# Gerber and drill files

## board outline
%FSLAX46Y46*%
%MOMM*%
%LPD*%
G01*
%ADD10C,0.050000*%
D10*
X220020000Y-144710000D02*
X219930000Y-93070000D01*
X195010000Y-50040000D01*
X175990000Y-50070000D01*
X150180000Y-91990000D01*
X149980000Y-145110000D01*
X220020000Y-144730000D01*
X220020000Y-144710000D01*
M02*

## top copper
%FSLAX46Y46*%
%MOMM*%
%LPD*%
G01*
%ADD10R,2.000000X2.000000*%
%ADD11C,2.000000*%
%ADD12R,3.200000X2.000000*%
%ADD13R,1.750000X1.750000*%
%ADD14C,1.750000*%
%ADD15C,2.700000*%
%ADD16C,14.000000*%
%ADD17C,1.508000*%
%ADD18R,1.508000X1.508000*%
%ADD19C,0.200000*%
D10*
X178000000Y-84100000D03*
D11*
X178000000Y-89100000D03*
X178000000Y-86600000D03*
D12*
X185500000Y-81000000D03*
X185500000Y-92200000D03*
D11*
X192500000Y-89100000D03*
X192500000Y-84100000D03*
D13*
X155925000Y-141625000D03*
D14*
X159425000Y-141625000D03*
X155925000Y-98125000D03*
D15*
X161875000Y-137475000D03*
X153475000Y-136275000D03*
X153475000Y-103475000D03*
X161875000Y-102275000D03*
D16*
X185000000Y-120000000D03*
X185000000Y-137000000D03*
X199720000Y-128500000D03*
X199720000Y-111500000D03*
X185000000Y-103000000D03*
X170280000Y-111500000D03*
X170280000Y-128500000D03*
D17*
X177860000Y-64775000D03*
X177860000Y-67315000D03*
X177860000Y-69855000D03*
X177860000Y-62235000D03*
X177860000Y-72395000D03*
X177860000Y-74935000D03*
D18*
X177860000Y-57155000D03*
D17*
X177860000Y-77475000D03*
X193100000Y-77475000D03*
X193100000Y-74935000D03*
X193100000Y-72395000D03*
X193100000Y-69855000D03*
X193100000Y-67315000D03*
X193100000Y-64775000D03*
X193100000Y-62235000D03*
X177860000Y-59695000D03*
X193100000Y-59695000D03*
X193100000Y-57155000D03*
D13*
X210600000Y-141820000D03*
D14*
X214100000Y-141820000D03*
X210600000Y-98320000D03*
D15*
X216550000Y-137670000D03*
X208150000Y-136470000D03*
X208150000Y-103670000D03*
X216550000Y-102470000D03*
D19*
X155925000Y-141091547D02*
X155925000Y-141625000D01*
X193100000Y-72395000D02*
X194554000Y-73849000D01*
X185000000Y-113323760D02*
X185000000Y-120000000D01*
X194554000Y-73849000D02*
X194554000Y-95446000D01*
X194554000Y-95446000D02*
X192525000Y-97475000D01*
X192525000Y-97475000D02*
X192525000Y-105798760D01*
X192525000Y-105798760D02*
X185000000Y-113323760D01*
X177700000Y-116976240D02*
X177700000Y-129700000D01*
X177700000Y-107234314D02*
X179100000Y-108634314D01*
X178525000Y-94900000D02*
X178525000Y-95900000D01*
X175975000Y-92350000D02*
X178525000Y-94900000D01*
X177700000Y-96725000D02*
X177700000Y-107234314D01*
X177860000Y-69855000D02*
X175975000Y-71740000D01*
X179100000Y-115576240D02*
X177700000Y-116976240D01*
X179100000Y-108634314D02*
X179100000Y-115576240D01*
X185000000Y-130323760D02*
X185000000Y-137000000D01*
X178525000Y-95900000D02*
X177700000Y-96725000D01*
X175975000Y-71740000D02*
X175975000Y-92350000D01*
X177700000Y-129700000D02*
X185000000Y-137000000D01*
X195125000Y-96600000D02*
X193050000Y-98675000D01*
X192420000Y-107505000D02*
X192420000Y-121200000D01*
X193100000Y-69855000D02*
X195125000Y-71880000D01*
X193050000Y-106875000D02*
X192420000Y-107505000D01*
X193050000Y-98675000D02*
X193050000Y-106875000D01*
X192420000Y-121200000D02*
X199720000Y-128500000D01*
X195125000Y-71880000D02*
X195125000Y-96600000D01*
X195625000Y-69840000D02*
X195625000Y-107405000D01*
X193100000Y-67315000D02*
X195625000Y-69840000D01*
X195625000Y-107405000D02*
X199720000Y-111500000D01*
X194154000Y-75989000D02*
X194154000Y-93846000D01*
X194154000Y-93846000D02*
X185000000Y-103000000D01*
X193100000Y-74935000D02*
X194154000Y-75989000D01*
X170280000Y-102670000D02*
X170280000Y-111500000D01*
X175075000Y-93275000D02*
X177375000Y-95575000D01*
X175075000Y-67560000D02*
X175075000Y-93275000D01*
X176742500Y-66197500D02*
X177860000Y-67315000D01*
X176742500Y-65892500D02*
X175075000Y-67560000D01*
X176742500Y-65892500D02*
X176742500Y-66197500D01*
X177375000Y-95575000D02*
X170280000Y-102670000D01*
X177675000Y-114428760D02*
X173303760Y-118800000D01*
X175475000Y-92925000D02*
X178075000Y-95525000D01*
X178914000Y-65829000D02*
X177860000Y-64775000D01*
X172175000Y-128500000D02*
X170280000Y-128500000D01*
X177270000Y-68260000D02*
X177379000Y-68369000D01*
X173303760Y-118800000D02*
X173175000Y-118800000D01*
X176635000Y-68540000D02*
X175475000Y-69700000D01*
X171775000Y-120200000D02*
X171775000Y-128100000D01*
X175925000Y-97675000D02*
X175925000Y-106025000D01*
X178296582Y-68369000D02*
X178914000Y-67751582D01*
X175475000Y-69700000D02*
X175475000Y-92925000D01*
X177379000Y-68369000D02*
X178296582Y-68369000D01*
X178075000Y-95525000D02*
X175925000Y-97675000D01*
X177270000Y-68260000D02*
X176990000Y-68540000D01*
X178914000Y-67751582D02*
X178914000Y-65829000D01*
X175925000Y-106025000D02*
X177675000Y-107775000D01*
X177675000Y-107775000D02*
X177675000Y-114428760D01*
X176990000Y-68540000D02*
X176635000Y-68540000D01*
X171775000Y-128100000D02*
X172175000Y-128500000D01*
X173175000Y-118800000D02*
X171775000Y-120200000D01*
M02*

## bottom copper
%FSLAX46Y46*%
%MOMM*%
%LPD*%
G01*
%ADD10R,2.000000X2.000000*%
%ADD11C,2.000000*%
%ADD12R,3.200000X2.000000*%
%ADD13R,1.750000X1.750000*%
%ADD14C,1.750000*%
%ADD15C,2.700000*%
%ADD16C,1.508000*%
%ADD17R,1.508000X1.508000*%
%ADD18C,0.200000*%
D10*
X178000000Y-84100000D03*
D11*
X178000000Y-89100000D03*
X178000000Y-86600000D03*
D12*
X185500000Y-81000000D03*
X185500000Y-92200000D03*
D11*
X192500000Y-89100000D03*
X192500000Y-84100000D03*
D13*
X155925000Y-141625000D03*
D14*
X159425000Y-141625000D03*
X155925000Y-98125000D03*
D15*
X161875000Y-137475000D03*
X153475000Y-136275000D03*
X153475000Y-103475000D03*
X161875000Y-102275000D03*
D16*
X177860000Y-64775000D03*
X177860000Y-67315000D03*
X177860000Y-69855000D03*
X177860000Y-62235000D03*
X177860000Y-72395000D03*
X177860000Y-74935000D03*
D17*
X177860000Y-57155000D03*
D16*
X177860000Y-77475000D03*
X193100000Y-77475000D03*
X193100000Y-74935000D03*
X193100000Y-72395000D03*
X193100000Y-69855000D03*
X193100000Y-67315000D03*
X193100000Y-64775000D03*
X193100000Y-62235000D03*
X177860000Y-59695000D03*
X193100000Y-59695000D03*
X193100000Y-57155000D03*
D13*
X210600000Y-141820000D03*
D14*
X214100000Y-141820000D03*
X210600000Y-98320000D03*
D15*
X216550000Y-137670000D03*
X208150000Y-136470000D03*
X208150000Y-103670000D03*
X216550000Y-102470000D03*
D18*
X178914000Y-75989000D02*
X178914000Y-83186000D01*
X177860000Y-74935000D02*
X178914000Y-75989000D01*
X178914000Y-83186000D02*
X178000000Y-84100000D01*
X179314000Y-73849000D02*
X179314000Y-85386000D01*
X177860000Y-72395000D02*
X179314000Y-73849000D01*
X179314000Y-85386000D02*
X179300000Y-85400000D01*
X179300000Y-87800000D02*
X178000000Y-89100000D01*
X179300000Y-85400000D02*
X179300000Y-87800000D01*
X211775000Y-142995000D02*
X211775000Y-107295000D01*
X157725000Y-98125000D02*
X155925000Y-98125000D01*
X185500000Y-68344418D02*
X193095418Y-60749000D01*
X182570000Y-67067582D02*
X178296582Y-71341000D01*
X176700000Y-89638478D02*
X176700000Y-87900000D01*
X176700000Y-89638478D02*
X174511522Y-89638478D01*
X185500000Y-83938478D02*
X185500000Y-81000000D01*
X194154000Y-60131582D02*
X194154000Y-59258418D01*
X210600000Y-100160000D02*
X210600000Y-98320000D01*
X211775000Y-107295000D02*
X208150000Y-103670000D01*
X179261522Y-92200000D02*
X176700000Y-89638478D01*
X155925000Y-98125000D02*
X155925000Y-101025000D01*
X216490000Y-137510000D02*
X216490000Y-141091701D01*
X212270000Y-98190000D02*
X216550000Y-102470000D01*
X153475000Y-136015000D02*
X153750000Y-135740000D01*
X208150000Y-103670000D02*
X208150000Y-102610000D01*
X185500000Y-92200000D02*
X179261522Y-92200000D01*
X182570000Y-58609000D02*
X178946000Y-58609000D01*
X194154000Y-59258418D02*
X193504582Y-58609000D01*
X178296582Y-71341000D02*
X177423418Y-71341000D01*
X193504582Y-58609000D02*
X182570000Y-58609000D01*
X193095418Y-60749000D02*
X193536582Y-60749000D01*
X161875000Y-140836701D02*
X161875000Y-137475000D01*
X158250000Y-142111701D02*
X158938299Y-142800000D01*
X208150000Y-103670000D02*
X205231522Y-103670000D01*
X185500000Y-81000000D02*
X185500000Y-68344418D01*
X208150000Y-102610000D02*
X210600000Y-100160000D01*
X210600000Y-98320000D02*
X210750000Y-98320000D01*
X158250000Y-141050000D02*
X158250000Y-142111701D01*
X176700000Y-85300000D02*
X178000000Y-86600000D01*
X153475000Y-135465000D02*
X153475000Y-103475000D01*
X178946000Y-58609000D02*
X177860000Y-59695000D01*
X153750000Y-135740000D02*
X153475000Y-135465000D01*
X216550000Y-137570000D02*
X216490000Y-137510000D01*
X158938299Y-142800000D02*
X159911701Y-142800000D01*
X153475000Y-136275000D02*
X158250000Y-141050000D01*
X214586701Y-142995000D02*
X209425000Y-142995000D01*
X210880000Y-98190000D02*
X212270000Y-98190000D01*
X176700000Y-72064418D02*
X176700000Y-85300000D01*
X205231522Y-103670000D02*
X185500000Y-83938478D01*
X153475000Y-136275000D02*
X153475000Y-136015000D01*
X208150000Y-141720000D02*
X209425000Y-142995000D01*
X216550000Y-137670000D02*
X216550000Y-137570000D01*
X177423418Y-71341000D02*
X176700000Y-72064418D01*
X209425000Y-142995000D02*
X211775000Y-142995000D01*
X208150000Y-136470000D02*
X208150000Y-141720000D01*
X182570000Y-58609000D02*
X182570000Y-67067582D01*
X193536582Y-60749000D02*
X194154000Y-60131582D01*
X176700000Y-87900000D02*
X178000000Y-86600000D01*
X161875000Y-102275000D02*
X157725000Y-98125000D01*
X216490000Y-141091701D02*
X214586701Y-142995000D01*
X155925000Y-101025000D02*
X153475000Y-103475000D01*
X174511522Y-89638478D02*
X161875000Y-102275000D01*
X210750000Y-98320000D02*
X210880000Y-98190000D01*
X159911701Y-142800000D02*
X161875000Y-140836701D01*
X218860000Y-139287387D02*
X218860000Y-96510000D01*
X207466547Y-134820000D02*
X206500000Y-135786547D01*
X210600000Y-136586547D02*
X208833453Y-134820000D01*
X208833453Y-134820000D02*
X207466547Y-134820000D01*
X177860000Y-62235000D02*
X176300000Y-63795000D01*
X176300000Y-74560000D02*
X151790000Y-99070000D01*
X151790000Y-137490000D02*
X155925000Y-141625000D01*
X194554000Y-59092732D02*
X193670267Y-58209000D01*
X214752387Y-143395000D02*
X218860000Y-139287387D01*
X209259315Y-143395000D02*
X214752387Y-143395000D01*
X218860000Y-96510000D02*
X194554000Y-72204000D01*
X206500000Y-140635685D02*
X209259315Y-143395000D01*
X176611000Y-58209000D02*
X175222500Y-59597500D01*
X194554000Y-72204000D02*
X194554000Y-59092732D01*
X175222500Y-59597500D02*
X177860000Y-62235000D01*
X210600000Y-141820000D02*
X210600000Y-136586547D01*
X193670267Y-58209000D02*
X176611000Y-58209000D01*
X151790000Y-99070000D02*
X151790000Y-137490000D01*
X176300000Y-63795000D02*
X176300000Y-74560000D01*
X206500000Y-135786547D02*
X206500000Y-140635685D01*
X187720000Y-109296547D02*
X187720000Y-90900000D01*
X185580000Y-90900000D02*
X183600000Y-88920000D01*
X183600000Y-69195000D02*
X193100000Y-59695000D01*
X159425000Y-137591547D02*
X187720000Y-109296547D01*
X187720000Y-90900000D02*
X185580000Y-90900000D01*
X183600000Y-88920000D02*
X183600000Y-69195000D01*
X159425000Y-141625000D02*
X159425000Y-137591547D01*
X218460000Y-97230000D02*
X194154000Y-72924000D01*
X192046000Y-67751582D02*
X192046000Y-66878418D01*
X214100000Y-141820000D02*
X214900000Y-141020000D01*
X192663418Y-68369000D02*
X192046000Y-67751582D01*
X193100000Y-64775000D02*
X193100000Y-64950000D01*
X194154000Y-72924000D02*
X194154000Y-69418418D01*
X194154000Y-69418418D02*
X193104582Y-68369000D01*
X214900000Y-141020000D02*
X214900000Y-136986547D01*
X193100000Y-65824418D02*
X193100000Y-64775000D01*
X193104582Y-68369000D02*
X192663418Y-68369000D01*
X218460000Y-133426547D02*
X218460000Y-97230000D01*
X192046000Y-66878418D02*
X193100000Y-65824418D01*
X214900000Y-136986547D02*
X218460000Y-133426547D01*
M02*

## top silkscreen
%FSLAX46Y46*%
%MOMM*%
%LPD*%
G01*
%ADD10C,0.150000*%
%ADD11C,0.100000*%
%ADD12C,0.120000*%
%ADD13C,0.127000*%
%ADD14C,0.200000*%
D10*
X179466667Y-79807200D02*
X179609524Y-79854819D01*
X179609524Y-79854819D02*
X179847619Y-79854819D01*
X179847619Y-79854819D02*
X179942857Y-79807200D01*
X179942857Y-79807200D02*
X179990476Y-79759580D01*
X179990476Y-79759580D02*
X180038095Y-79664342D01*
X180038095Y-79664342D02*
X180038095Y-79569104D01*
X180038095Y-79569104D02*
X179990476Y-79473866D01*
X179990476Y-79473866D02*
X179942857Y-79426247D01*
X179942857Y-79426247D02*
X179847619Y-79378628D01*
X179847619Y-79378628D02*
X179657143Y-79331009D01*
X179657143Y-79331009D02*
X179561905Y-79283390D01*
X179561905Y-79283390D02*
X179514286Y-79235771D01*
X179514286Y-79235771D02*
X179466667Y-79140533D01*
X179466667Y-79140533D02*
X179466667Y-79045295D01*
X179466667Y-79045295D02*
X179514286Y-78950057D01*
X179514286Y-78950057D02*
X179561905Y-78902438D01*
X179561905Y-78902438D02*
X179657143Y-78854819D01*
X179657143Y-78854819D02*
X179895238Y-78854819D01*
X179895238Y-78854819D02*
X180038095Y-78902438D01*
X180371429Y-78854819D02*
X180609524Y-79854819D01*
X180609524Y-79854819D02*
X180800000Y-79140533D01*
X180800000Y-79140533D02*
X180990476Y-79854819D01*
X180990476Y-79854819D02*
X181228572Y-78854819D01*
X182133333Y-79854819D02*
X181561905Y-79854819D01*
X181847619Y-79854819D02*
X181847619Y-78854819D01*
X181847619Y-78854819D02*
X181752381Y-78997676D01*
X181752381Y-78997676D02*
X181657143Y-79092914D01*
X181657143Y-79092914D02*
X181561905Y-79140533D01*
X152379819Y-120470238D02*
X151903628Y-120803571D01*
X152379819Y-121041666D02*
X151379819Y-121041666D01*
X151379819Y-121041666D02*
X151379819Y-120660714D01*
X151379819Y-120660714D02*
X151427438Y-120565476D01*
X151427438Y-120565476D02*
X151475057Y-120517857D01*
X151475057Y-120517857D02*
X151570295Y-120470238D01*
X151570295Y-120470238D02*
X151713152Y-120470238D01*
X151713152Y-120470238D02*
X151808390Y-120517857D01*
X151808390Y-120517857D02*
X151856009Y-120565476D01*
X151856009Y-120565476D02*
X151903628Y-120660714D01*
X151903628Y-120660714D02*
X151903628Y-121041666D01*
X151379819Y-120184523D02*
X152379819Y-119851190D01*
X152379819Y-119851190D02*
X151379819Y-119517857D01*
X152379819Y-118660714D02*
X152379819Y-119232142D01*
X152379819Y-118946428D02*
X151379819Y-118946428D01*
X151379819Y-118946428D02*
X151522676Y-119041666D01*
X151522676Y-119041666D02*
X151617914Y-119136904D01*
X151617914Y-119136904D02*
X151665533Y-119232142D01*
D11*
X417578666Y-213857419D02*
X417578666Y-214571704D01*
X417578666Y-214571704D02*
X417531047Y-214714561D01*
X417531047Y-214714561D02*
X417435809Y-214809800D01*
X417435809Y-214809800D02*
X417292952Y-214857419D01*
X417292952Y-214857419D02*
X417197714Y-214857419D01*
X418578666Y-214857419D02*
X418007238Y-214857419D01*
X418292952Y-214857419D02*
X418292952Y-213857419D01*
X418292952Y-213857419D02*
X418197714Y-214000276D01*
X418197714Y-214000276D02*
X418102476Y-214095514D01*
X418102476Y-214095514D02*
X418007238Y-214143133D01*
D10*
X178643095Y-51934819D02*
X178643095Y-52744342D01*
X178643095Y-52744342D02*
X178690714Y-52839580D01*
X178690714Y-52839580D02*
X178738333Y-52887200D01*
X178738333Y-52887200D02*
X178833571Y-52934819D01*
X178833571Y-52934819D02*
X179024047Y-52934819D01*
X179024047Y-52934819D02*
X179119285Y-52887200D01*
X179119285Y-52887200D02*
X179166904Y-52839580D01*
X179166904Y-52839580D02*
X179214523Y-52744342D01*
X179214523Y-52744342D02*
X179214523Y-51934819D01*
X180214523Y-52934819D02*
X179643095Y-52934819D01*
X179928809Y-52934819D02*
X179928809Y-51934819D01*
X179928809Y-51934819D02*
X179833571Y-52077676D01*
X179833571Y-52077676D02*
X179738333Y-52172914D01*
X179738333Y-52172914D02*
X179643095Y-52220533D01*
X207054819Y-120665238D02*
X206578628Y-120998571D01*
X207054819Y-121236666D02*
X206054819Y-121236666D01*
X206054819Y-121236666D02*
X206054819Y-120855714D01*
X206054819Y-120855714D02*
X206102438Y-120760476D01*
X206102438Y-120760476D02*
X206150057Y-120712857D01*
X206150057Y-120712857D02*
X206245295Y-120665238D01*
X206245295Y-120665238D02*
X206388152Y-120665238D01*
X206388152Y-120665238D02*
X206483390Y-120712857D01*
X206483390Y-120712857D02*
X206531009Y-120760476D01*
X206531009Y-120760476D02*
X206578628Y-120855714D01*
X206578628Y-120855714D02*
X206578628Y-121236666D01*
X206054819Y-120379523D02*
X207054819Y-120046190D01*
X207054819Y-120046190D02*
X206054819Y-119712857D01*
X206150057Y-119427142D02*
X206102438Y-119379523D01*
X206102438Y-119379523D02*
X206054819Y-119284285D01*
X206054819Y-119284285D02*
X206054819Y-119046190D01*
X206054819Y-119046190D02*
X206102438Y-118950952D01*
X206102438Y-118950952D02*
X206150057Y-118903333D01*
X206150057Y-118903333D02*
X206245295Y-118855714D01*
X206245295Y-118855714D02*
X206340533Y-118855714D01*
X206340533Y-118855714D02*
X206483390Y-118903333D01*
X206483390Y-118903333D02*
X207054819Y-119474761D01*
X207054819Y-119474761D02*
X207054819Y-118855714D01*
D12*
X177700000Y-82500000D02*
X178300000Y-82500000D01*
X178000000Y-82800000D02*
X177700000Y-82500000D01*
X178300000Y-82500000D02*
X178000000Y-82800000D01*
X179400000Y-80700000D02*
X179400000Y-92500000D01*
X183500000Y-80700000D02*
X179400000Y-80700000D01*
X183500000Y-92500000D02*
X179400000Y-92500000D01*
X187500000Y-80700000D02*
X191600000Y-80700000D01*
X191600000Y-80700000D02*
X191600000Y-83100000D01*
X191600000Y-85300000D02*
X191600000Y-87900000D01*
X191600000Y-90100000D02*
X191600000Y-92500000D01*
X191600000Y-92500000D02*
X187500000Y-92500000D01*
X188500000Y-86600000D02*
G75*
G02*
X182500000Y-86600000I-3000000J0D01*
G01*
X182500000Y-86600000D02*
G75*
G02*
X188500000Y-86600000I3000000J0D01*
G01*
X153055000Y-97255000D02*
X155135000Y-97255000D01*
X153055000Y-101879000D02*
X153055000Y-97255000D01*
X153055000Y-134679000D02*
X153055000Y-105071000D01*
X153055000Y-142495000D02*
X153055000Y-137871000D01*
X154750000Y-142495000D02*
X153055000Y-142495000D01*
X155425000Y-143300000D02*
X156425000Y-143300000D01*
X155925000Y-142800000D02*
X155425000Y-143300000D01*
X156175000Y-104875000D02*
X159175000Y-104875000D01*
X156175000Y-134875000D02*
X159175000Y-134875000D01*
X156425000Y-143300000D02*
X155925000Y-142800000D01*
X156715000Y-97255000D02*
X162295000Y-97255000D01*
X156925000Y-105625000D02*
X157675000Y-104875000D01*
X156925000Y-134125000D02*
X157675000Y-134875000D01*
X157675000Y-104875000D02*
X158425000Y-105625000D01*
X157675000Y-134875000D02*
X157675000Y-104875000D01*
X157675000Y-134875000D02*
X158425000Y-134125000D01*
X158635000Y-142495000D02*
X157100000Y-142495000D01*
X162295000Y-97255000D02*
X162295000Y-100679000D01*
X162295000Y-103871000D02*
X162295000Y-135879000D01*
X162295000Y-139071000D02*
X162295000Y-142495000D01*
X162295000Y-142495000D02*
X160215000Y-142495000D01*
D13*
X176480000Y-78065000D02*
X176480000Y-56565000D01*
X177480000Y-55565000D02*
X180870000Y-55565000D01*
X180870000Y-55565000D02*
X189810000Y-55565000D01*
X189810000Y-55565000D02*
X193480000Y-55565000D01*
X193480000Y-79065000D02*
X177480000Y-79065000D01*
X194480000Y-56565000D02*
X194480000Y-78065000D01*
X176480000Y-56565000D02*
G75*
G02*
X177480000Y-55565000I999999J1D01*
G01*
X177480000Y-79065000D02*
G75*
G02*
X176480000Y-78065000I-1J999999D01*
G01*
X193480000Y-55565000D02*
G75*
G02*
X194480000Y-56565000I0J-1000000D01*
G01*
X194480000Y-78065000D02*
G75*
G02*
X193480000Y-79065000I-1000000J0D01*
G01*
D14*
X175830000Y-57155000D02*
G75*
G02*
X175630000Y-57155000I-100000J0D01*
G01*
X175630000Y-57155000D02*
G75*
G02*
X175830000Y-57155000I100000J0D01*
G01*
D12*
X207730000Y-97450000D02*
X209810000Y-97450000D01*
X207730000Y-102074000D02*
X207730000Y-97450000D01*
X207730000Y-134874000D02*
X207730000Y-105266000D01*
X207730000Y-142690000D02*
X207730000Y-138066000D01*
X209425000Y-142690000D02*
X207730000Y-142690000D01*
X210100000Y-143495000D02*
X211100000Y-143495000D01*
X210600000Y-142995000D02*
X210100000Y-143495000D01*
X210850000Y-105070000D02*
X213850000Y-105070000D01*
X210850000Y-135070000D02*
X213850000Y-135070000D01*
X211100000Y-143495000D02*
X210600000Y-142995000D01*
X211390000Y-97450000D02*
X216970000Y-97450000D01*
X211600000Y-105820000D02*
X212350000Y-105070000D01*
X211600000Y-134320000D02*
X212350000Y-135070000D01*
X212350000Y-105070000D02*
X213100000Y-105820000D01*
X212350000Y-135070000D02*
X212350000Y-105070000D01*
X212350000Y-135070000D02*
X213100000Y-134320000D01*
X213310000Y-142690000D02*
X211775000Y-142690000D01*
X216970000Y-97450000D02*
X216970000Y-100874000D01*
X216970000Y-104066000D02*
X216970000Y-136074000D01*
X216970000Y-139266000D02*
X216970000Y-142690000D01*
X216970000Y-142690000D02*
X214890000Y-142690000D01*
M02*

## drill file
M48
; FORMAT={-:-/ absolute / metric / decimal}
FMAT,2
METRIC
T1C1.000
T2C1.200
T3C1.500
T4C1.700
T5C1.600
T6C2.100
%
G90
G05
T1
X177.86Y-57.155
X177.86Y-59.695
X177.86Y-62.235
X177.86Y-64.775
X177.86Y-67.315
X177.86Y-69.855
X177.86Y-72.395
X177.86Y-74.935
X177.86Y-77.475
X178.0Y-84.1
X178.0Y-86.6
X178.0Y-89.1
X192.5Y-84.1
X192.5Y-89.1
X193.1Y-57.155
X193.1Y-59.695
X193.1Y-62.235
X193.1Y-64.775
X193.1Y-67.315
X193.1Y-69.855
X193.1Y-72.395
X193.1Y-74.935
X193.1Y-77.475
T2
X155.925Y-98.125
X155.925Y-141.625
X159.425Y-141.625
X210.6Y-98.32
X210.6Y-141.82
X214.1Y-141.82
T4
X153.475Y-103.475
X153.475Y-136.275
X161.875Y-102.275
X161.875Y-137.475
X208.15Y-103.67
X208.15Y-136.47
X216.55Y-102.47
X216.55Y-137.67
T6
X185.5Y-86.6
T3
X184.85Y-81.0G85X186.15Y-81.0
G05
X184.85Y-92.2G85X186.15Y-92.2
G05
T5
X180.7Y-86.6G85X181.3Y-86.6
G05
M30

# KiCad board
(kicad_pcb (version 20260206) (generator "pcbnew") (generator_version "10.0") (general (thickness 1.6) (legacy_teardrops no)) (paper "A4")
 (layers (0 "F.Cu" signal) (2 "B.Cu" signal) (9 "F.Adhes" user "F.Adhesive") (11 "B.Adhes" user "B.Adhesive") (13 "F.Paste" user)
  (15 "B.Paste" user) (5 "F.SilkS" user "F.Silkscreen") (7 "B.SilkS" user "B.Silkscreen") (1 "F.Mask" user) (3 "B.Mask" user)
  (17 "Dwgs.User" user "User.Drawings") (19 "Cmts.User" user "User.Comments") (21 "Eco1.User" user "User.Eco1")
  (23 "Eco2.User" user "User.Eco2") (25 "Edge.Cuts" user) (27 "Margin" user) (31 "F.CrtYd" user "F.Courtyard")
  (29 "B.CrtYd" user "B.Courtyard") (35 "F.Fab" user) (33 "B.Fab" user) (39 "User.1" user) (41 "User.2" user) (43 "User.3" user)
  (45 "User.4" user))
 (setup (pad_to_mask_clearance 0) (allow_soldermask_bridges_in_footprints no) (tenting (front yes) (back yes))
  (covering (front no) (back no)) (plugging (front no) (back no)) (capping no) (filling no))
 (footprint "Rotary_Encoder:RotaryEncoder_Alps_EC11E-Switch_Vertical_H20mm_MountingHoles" (layer "F.Cu") (at 178 84.1)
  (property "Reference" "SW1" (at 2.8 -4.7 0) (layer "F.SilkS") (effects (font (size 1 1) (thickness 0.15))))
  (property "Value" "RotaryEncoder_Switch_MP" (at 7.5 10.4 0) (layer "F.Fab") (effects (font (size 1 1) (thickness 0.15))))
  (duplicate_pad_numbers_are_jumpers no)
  (fp_line (start -0.3 -1.6) (end 0.3 -1.6) (stroke (width 0.12) (type solid)) (layer "F.SilkS"))
  (fp_line (start 0 -1.3) (end -0.3 -1.6) (stroke (width 0.12) (type solid)) (layer "F.SilkS"))
  (fp_line (start 0.3 -1.6) (end 0 -1.3) (stroke (width 0.12) (type solid)) (layer "F.SilkS"))
  (fp_line (start 1.4 -3.4) (end 1.4 8.4) (stroke (width 0.12) (type solid)) (layer "F.SilkS"))
  (fp_line (start 5.5 -3.4) (end 1.4 -3.4) (stroke (width 0.12) (type solid)) (layer "F.SilkS"))
  (fp_line (start 5.5 8.4) (end 1.4 8.4) (stroke (width 0.12) (type solid)) (layer "F.SilkS"))
  (fp_line (start 9.5 -3.4) (end 13.6 -3.4) (stroke (width 0.12) (type solid)) (layer "F.SilkS"))
  (fp_line (start 13.6 -3.4) (end 13.6 -1) (stroke (width 0.12) (type solid)) (layer "F.SilkS"))
  (fp_line (start 13.6 1.2) (end 13.6 3.8) (stroke (width 0.12) (type solid)) (layer "F.SilkS"))
  (fp_line (start 13.6 6) (end 13.6 8.4) (stroke (width 0.12) (type solid)) (layer "F.SilkS"))
  (fp_line (start 13.6 8.4) (end 9.5 8.4) (stroke (width 0.12) (type solid)) (layer "F.SilkS"))
  (fp_circle (center 7.5 2.5) (end 10.5 2.5) (stroke (width 0.12) (type solid)) (fill no) (layer "F.SilkS"))
  (pad "" np_thru_hole oval (at 3 2.5) (size 2.2 1.6) (drill oval 2.2 1.6) (layers "*.Mask"))
  (pad "" np_thru_hole circle (at 7.5 2.5) (size 2.1 2.1) (drill 2.1) (layers "*.Mask"))
  (pad "A" thru_hole rect (at 0 0) (size 2 2) (drill 1) (layers "*.Cu" "*.Mask") (remove_unused_layers no) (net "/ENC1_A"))
  (pad "B" thru_hole circle (at 0 5) (size 2 2) (drill 1) (layers "*.Cu" "*.Mask") (remove_unused_layers no) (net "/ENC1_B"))
  (pad "C" thru_hole circle (at 0 2.5) (size 2 2) (drill 1) (layers "*.Cu" "*.Mask") (remove_unused_layers no) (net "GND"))
  (pad "MP" thru_hole rect (at 7.5 -3.1) (size 3.2 2) (drill oval 2.8 1.5) (layers "*.Cu" "*.Mask") (remove_unused_layers no) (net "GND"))
  (pad "MP" thru_hole rect (at 7.5 8.1) (size 3.2 2) (drill oval 2.8 1.5) (layers "*.Cu" "*.Mask") (remove_unused_layers no) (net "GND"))
  (pad "S1" thru_hole circle (at 14.5 5) (size 2 2) (drill 1) (layers "*.Cu" "*.Mask") (remove_unused_layers no)
   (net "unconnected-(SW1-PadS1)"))
  (pad "S2" thru_hole circle (at 14.5 0) (size 2 2) (drill 1) (layers "*.Cu" "*.Mask") (remove_unused_layers no)
   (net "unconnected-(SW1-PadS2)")))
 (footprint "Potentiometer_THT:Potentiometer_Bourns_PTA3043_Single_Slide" (layer "F.Cu") (at 155.925 141.625 90)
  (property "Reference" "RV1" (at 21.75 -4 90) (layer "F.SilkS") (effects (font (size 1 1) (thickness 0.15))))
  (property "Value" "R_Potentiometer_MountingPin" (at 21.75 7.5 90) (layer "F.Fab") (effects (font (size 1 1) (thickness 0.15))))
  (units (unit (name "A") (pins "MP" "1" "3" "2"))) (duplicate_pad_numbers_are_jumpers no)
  (fp_line (start 44.37 -2.87) (end 44.37 -0.79) (stroke (width 0.12) (type solid)) (layer "F.SilkS"))
  (fp_line (start 39.746 -2.87) (end 44.37 -2.87) (stroke (width 0.12) (type solid)) (layer "F.SilkS"))
  (fp_line (start 6.946 -2.87) (end 36.554 -2.87) (stroke (width 0.12) (type solid)) (layer "F.SilkS"))
  (fp_line (start -0.87 -2.87) (end 3.754 -2.87) (stroke (width 0.12) (type solid)) (layer "F.SilkS"))
  (fp_line (start -0.87 -1.175) (end -0.87 -2.87) (stroke (width 0.12) (type solid)) (layer "F.SilkS"))
  (fp_line (start -1.675 -0.5) (end -1.675 0.5) (stroke (width 0.12) (type solid)) (layer "F.SilkS"))
  (fp_line (start -1.175 0) (end -1.675 -0.5) (stroke (width 0.12) (type solid)) (layer "F.SilkS"))
  (fp_line (start 36.75 0.25) (end 36.75 3.25) (stroke (width 0.12) (type solid)) (layer "F.SilkS"))
  (fp_line (start 6.75 0.25) (end 6.75 3.25) (stroke (width 0.12) (type solid)) (layer "F.SilkS"))
  (fp_line (start -1.675 0.5) (end -1.175 0) (stroke (width 0.12) (type solid)) (layer "F.SilkS"))
  (fp_line (start 44.37 0.79) (end 44.37 6.37) (stroke (width 0.12) (type solid)) (layer "F.SilkS"))
  (fp_line (start 36 1) (end 36.75 1.75) (stroke (width 0.12) (type solid)) (layer "F.SilkS"))
  (fp_line (start 7.5 1) (end 6.75 1.75) (stroke (width 0.12) (type solid)) (layer "F.SilkS"))
  (fp_line (start 36.75 1.75) (end 36 2.5) (stroke (width 0.12) (type solid)) (layer "F.SilkS"))
  (fp_line (start 6.75 1.75) (end 36.75 1.75) (stroke (width 0.12) (type solid)) (layer "F.SilkS"))
  (fp_line (start 6.75 1.75) (end 7.5 2.5) (stroke (width 0.12) (type solid)) (layer "F.SilkS"))
  (fp_line (start -0.87 2.71) (end -0.87 1.175) (stroke (width 0.12) (type solid)) (layer "F.SilkS"))
  (fp_line (start 44.37 6.37) (end 40.946 6.37) (stroke (width 0.12) (type solid)) (layer "F.SilkS"))
  (fp_line (start 37.754 6.37) (end 5.746 6.37) (stroke (width 0.12) (type solid)) (layer "F.SilkS"))
  (fp_line (start 2.554 6.37) (end -0.87 6.37) (stroke (width 0.12) (type solid)) (layer "F.SilkS"))
  (fp_line (start -0.87 6.37) (end -0.87 4.29) (stroke (width 0.12) (type solid)) (layer "F.SilkS"))
  (pad "1" thru_hole rect (at 0 0 90) (size 1.75 1.75) (drill 1.2) (layers "*.Cu" "*.Mask") (remove_unused_layers no) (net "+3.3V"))
  (pad "2" thru_hole circle (at 0 3.5 90) (size 1.75 1.75) (drill 1.2) (layers "*.Cu" "*.Mask") (remove_unused_layers no) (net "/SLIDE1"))
  (pad "3" thru_hole circle (at 43.5 0 90) (size 1.75 1.75) (drill 1.2) (layers "*.Cu" "*.Mask") (remove_unused_layers no) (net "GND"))
  (pad "MP" thru_hole circle (at 4.15 5.95 90) (size 2.7 2.7) (drill 1.7) (layers "*.Cu" "*.Mask") (remove_unused_layers no) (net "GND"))
  (pad "MP" thru_hole circle (at 5.35 -2.45 90) (size 2.7 2.7) (drill 1.7) (layers "*.Cu" "*.Mask") (remove_unused_layers no) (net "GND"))
  (pad "MP" thru_hole circle (at 38.15 -2.45 90) (size 2.7 2.7) (drill 1.7) (layers "*.Cu" "*.Mask") (remove_unused_layers no) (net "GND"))
  (pad "MP" thru_hole circle (at 39.35 5.95 90) (size 2.7 2.7) (drill 1.7) (layers "*.Cu" "*.Mask") (remove_unused_layers no) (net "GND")))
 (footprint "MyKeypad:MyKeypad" (layer "F.Cu") (at 407 226)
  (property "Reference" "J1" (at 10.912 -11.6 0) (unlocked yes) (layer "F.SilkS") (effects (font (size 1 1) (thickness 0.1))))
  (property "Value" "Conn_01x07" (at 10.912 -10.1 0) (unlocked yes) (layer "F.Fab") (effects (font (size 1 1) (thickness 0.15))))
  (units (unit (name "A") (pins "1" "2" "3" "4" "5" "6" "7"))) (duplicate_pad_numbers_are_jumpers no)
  (pad "1" smd circle (at -222 -106 120) (size 14 14) (layers "F.Cu" "F.Mask") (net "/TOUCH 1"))
  (pad "2" smd circle (at -222 -89 120) (size 14 14) (layers "F.Cu" "F.Mask") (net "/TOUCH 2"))
  (pad "3" smd circle (at -207.28 -97.5 120) (size 14 14) (layers "F.Cu" "F.Mask") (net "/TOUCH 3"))
  (pad "4" smd circle (at -207.28 -114.5 120) (size 14 14) (layers "F.Cu" "F.Mask") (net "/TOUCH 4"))
  (pad "5" smd circle (at -222 -123 120) (size 14 14) (layers "F.Cu" "F.Mask") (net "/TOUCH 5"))
  (pad "6" smd circle (at -236.72 -114.5 120) (size 14 14) (layers "F.Cu" "F.Mask") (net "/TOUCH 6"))
  (pad "7" smd circle (at -236.72 -97.5 120) (size 14 14) (layers "F.Cu" "F.Mask") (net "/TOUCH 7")))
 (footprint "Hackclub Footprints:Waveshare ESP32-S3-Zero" (layer "F.Cu") (at 185.48 67.315)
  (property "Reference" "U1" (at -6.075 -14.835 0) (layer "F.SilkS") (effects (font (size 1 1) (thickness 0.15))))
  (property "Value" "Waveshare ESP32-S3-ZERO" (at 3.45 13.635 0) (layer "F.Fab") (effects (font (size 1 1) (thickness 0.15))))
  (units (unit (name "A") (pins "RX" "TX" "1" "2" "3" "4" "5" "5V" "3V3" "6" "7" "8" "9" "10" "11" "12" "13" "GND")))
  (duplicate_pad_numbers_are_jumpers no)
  (fp_line (start -9 10.75) (end -9 -10.75) (stroke (width 0.127) (type solid)) (layer "F.SilkS"))
  (fp_line (start -8 -11.75) (end -4.61 -11.75) (stroke (width 0.127) (type solid)) (layer "F.SilkS"))
  (fp_line (start -4.61 -11.75) (end 4.33 -11.75) (stroke (width 0.127) (type solid)) (layer "F.SilkS"))
  (fp_line (start 4.33 -11.75) (end 8 -11.75) (stroke (width 0.127) (type solid)) (layer "F.SilkS"))
  (fp_line (start 8 11.75) (end -8 11.75) (stroke (width 0.127) (type solid)) (layer "F.SilkS"))
  (fp_line (start 9 -10.75) (end 9 10.75) (stroke (width 0.127) (type solid)) (layer "F.SilkS"))
  (fp_arc (start -9 -10.75) (mid -8.707107 -11.457107) (end -8 -11.75) (stroke (width 0.127) (type solid)) (layer "F.SilkS"))
  (fp_arc (start -8 11.75) (mid -8.707107 11.457107) (end -9 10.75) (stroke (width 0.127) (type solid)) (layer "F.SilkS"))
  (fp_arc (start 8 -11.75) (mid 8.707107 -11.457107) (end 9 -10.75) (stroke (width 0.127) (type solid)) (layer "F.SilkS"))
  (fp_arc (start 9 10.75) (mid 8.707107 11.457107) (end 8 11.75) (stroke (width 0.127) (type solid)) (layer "F.SilkS"))
  (fp_circle (center -9.75 -10.16) (end -9.65 -10.16) (stroke (width 0.2) (type solid)) (fill no) (layer "F.SilkS"))
  (pad "1" thru_hole circle (at -7.62 -2.54) (size 1.508 1.508) (drill 1) (layers "*.Cu" "*.Mask") (remove_unused_layers no)
   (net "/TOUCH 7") (solder_mask_margin 0.102))
  (pad "2" thru_hole circle (at -7.62 0) (size 1.508 1.508) (drill 1) (layers "*.Cu" "*.Mask") (remove_unused_layers no) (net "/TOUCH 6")
   (solder_mask_margin 0.102))
  (pad "3" thru_hole circle (at -7.62 2.54) (size 1.508 1.508) (drill 1) (layers "*.Cu" "*.Mask") (remove_unused_layers no) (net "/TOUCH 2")
   (solder_mask_margin 0.102))
  (pad "3V3" thru_hole circle (at -7.62 -5.08) (size 1.508 1.508) (drill 1) (layers "*.Cu" "*.Mask") (remove_unused_layers no) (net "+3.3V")
   (solder_mask_margin 0.102))
  (pad "4" thru_hole circle (at -7.62 5.08) (size 1.508 1.508) (drill 1) (layers "*.Cu" "*.Mask") (remove_unused_layers no) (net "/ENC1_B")
   (solder_mask_margin 0.102))
  (pad "5" thru_hole circle (at -7.62 7.62) (size 1.508 1.508) (drill 1) (layers "*.Cu" "*.Mask") (remove_unused_layers no) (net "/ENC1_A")
   (solder_mask_margin 0.102))
  (pad "5V" thru_hole rect (at -7.62 -10.16) (size 1.508 1.508) (drill 1) (layers "*.Cu" "*.Mask") (remove_unused_layers no) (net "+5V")
   (solder_mask_margin 0.102))
  (pad "6" thru_hole circle (at -7.62 10.16) (size 1.508 1.508) (drill 1) (layers "*.Cu" "*.Mask") (remove_unused_layers no)
   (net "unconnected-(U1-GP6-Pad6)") (solder_mask_margin 0.102))
  (pad "7" thru_hole circle (at 7.62 10.16) (size 1.508 1.508) (drill 1) (layers "*.Cu" "*.Mask") (remove_unused_layers no)
   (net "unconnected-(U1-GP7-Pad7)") (solder_mask_margin 0.102))
  (pad "8" thru_hole circle (at 7.62 7.62) (size 1.508 1.508) (drill 1) (layers "*.Cu" "*.Mask") (remove_unused_layers no) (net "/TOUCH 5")
   (solder_mask_margin 0.102))
  (pad "9" thru_hole circle (at 7.62 5.08) (size 1.508 1.508) (drill 1) (layers "*.Cu" "*.Mask") (remove_unused_layers no) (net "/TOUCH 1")
   (solder_mask_margin 0.102))
  (pad "10" thru_hole circle (at 7.62 2.54) (size 1.508 1.508) (drill 1) (layers "*.Cu" "*.Mask") (remove_unused_layers no) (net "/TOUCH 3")
   (solder_mask_margin 0.102))
  (pad "11" thru_hole circle (at 7.62 0) (size 1.508 1.508) (drill 1) (layers "*.Cu" "*.Mask") (remove_unused_layers no) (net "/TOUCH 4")
   (solder_mask_margin 0.102))
  (pad "12" thru_hole circle (at 7.62 -2.54) (size 1.508 1.508) (drill 1) (layers "*.Cu" "*.Mask") (remove_unused_layers no) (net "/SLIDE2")
   (solder_mask_margin 0.102))
  (pad "13" thru_hole circle (at 7.62 -5.08) (size 1.508 1.508) (drill 1) (layers "*.Cu" "*.Mask") (remove_unused_layers no)
   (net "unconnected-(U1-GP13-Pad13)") (solder_mask_margin 0.102))
  (pad "GND" thru_hole circle (at -7.62 -7.62) (size 1.508 1.508) (drill 1) (layers "*.Cu" "*.Mask") (remove_unused_layers no) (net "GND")
   (solder_mask_margin 0.102))
  (pad "RX" thru_hole circle (at 7.62 -7.62) (size 1.508 1.508) (drill 1) (layers "*.Cu" "*.Mask") (remove_unused_layers no) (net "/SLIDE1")
   (solder_mask_margin 0.102))
  (pad "TX" thru_hole circle (at 7.62 -10.16) (size 1.508 1.508) (drill 1) (layers "*.Cu" "*.Mask") (remove_unused_layers no)
   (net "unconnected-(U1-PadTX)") (solder_mask_margin 0.102)))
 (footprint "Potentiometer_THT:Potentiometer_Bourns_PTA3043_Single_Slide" (layer "F.Cu") (at 210.6 141.82 90)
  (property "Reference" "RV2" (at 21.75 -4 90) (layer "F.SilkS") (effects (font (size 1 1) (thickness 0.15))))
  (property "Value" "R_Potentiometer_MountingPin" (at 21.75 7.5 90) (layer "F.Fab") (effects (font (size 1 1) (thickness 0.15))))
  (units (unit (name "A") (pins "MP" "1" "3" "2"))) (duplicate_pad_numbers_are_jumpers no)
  (fp_line (start 44.37 -2.87) (end 44.37 -0.79) (stroke (width 0.12) (type solid)) (layer "F.SilkS"))
  (fp_line (start 39.746 -2.87) (end 44.37 -2.87) (stroke (width 0.12) (type solid)) (layer "F.SilkS"))
  (fp_line (start 6.946 -2.87) (end 36.554 -2.87) (stroke (width 0.12) (type solid)) (layer "F.SilkS"))
  (fp_line (start -0.87 -2.87) (end 3.754 -2.87) (stroke (width 0.12) (type solid)) (layer "F.SilkS"))
  (fp_line (start -0.87 -1.175) (end -0.87 -2.87) (stroke (width 0.12) (type solid)) (layer "F.SilkS"))
  (fp_line (start -1.675 -0.5) (end -1.675 0.5) (stroke (width 0.12) (type solid)) (layer "F.SilkS"))
  (fp_line (start -1.175 0) (end -1.675 -0.5) (stroke (width 0.12) (type solid)) (layer "F.SilkS"))
  (fp_line (start 36.75 0.25) (end 36.75 3.25) (stroke (width 0.12) (type solid)) (layer "F.SilkS"))
  (fp_line (start 6.75 0.25) (end 6.75 3.25) (stroke (width 0.12) (type solid)) (layer "F.SilkS"))
  (fp_line (start -1.675 0.5) (end -1.175 0) (stroke (width 0.12) (type solid)) (layer "F.SilkS"))
  (fp_line (start 44.37 0.79) (end 44.37 6.37) (stroke (width 0.12) (type solid)) (layer "F.SilkS"))
  (fp_line (start 36 1) (end 36.75 1.75) (stroke (width 0.12) (type solid)) (layer "F.SilkS"))
  (fp_line (start 7.5 1) (end 6.75 1.75) (stroke (width 0.12) (type solid)) (layer "F.SilkS"))
  (fp_line (start 36.75 1.75) (end 36 2.5) (stroke (width 0.12) (type solid)) (layer "F.SilkS"))
  (fp_line (start 6.75 1.75) (end 36.75 1.75) (stroke (width 0.12) (type solid)) (layer "F.SilkS"))
  (fp_line (start 6.75 1.75) (end 7.5 2.5) (stroke (width 0.12) (type solid)) (layer "F.SilkS"))
  (fp_line (start -0.87 2.71) (end -0.87 1.175) (stroke (width 0.12) (type solid)) (layer "F.SilkS"))
  (fp_line (start 44.37 6.37) (end 40.946 6.37) (stroke (width 0.12) (type solid)) (layer "F.SilkS"))
  (fp_line (start 37.754 6.37) (end 5.746 6.37) (stroke (width 0.12) (type solid)) (layer "F.SilkS"))
  (fp_line (start 2.554 6.37) (end -0.87 6.37) (stroke (width 0.12) (type solid)) (layer "F.SilkS"))
  (fp_line (start -0.87 6.37) (end -0.87 4.29) (stroke (width 0.12) (type solid)) (layer "F.SilkS"))
  (pad "1" thru_hole rect (at 0 0 90) (size 1.75 1.75) (drill 1.2) (layers "*.Cu" "*.Mask") (remove_unused_layers no) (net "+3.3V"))
  (pad "2" thru_hole circle (at 0 3.5 90) (size 1.75 1.75) (drill 1.2) (layers "*.Cu" "*.Mask") (remove_unused_layers no) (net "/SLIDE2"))
  (pad "3" thru_hole circle (at 43.5 0 90) (size 1.75 1.75) (drill 1.2) (layers "*.Cu" "*.Mask") (remove_unused_layers no) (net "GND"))
  (pad "MP" thru_hole circle (at 4.15 5.95 90) (size 2.7 2.7) (drill 1.7) (layers "*.Cu" "*.Mask") (remove_unused_layers no) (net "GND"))
  (pad "MP" thru_hole circle (at 5.35 -2.45 90) (size 2.7 2.7) (drill 1.7) (layers "*.Cu" "*.Mask") (remove_unused_layers no) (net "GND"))
  (pad "MP" thru_hole circle (at 38.15 -2.45 90) (size 2.7 2.7) (drill 1.7) (layers "*.Cu" "*.Mask") (remove_unused_layers no) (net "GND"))
  (pad "MP" thru_hole circle (at 39.35 5.95 90) (size 2.7 2.7) (drill 1.7) (layers "*.Cu" "*.Mask") (remove_unused_layers no) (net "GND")))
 (gr_poly
  (pts (xy 220.02 144.71) (xy 219.93 93.07) (xy 195.01 50.04) (xy 175.99 50.07) (xy 150.18 91.99) (xy 149.98 145.11) (xy 220.02 144.73))
  (stroke (width 0.05) (type solid)) (fill no) (layer "Edge.Cuts"))
 (segment (start 178.914 75.989) (end 178.914 83.186) (width 0.2) (layer "B.Cu") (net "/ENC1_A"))
 (segment (start 177.86 74.935) (end 178.914 75.989) (width 0.2) (layer "B.Cu") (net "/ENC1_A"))
 (segment (start 178.914 83.186) (end 178 84.1) (width 0.2) (layer "B.Cu") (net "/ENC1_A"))
 (segment (start 179.314 73.849) (end 179.314 85.386) (width 0.2) (layer "B.Cu") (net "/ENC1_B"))
 (segment (start 177.86 72.395) (end 179.314 73.849) (width 0.2) (layer "B.Cu") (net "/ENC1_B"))
 (segment (start 179.314 85.386) (end 179.3 85.4) (width 0.2) (layer "B.Cu") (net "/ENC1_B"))
 (segment (start 179.3 87.8) (end 178 89.1) (width 0.2) (layer "B.Cu") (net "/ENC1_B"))
 (segment (start 179.3 85.4) (end 179.3 87.8) (width 0.2) (layer "B.Cu") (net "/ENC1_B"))
 (segment (start 211.775 142.995) (end 211.775 107.295) (width 0.2) (layer "B.Cu") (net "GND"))
 (segment (start 157.725 98.125) (end 155.925 98.125) (width 0.2) (layer "B.Cu") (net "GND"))
 (segment (start 185.5 68.344418) (end 193.095418 60.749) (width 0.2) (layer "B.Cu") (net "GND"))
 (segment (start 182.57 67.067582) (end 178.296582 71.341) (width 0.2) (layer "B.Cu") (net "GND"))
 (segment (start 176.7 89.638478) (end 176.7 87.9) (width 0.2) (layer "B.Cu") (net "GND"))
 (segment (start 176.7 89.638478) (end 174.511522 89.638478) (width 0.2) (layer "B.Cu") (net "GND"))
 (segment (start 185.5 83.938478) (end 185.5 81) (width 0.2) (layer "B.Cu") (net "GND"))
 (segment (start 194.154 60.131582) (end 194.154 59.258418) (width 0.2) (layer "B.Cu") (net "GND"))
 (segment (start 210.6 100.16) (end 210.6 98.32) (width 0.2) (layer "B.Cu") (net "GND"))
 (segment (start 211.775 107.295) (end 208.15 103.67) (width 0.2) (layer "B.Cu") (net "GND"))
 (segment (start 179.261522 92.2) (end 176.7 89.638478) (width 0.2) (layer "B.Cu") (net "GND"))
 (segment (start 155.925 98.125) (end 155.925 101.025) (width 0.2) (layer "B.Cu") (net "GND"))
 (segment (start 216.49 137.51) (end 216.49 141.091701) (width 0.2) (layer "B.Cu") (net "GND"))
 (segment (start 212.27 98.19) (end 216.55 102.47) (width 0.2) (layer "B.Cu") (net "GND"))
 (segment (start 153.475 136.015) (end 153.75 135.74) (width 0.2) (layer "B.Cu") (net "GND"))
 (segment (start 208.15 103.67) (end 208.15 102.61) (width 0.2) (layer "B.Cu") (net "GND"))
 (segment (start 185.5 92.2) (end 179.261522 92.2) (width 0.2) (layer "B.Cu") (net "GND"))
 (segment (start 182.57 58.609) (end 178.946 58.609) (width 0.2) (layer "B.Cu") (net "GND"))
 (segment (start 194.154 59.258418) (end 193.504582 58.609) (width 0.2) (layer "B.Cu") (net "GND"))
 (segment (start 178.296582 71.341) (end 177.423418 71.341) (width 0.2) (layer "B.Cu") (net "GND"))
 (segment (start 193.504582 58.609) (end 182.57 58.609) (width 0.2) (layer "B.Cu") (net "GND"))
 (segment (start 193.095418 60.749) (end 193.536582 60.749) (width 0.2) (layer "B.Cu") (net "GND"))
 (segment (start 161.875 140.836701) (end 161.875 137.475) (width 0.2) (layer "B.Cu") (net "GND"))
 (segment (start 158.25 142.111701) (end 158.938299 142.8) (width 0.2) (layer "B.Cu") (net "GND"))
 (segment (start 208.15 103.67) (end 205.231522 103.67) (width 0.2) (layer "B.Cu") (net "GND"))
 (segment (start 185.5 81) (end 185.5 68.344418) (width 0.2) (layer "B.Cu") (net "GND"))
 (segment (start 208.15 102.61) (end 210.6 100.16) (width 0.2) (layer "B.Cu") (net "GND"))
 (segment (start 210.6 98.32) (end 210.75 98.32) (width 0.2) (layer "B.Cu") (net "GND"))
 (segment (start 158.25 141.05) (end 158.25 142.111701) (width 0.2) (layer "B.Cu") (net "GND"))
 (segment (start 176.7 85.3) (end 178 86.6) (width 0.2) (layer "B.Cu") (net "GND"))
 (segment (start 153.475 135.465) (end 153.475 103.475) (width 0.2) (layer "B.Cu") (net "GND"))
 (segment (start 178.946 58.609) (end 177.86 59.695) (width 0.2) (layer "B.Cu") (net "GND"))
 (segment (start 153.75 135.74) (end 153.475 135.465) (width 0.2) (layer "B.Cu") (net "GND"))
 (segment (start 216.55 137.57) (end 216.49 137.51) (width 0.2) (layer "B.Cu") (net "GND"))
 (segment (start 158.938299 142.8) (end 159.911701 142.8) (width 0.2) (layer "B.Cu") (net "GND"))
 (segment (start 153.475 136.275) (end 158.25 141.05) (width 0.2) (layer "B.Cu") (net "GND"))
 (segment (start 214.586701 142.995) (end 209.425 142.995) (width 0.2) (layer "B.Cu") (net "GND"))
 (segment (start 210.88 98.19) (end 212.27 98.19) (width 0.2) (layer "B.Cu") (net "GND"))
 (segment (start 176.7 72.064418) (end 176.7 85.3) (width 0.2) (layer "B.Cu") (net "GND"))
 (segment (start 205.231522 103.67) (end 185.5 83.938478) (width 0.2) (layer "B.Cu") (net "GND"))
 (segment (start 153.475 136.275) (end 153.475 136.015) (width 0.2) (layer "B.Cu") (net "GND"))
 (segment (start 208.15 141.72) (end 209.425 142.995) (width 0.2) (layer "B.Cu") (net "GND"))
 (segment (start 216.55 137.67) (end 216.55 137.57) (width 0.2) (layer "B.Cu") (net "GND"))
 (segment (start 177.423418 71.341) (end 176.7 72.064418) (width 0.2) (layer "B.Cu") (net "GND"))
 (segment (start 209.425 142.995) (end 211.775 142.995) (width 0.2) (layer "B.Cu") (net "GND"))
 (segment (start 208.15 136.47) (end 208.15 141.72) (width 0.2) (layer "B.Cu") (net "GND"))
 (segment (start 182.57 58.609) (end 182.57 67.067582) (width 0.2) (layer "B.Cu") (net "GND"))
 (segment (start 193.536582 60.749) (end 194.154 60.131582) (width 0.2) (layer "B.Cu") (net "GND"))
 (segment (start 176.7 87.9) (end 178 86.6) (width 0.2) (layer "B.Cu") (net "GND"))
 (segment (start 161.875 102.275) (end 157.725 98.125) (width 0.2) (layer "B.Cu") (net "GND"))
 (segment (start 216.49 141.091701) (end 214.586701 142.995) (width 0.2) (layer "B.Cu") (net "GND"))
 (segment (start 155.925 101.025) (end 153.475 103.475) (width 0.2) (layer "B.Cu") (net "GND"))
 (segment (start 174.511522 89.638478) (end 161.875 102.275) (width 0.2) (layer "B.Cu") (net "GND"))
 (segment (start 210.75 98.32) (end 210.88 98.19) (width 0.2) (layer "B.Cu") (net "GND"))
 (segment (start 159.911701 142.8) (end 161.875 140.836701) (width 0.2) (layer "B.Cu") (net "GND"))
 (segment (start 155.925 141.091547) (end 155.925 141.625) (width 0.2) (layer "F.Cu") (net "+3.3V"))
 (segment (start 218.86 139.287387) (end 218.86 96.51) (width 0.2) (layer "B.Cu") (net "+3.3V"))
 (segment (start 207.466547 134.82) (end 206.5 135.786547) (width 0.2) (layer "B.Cu") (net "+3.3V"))
 (segment (start 210.6 136.586547) (end 208.833453 134.82) (width 0.2) (layer "B.Cu") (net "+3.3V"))
 (segment (start 208.833453 134.82) (end 207.466547 134.82) (width 0.2) (layer "B.Cu") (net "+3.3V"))
 (segment (start 177.86 62.235) (end 176.3 63.795) (width 0.2) (layer "B.Cu") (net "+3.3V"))
 (segment (start 176.3 74.56) (end 151.79 99.07) (width 0.2) (layer "B.Cu") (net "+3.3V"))
 (segment (start 151.79 137.49) (end 155.925 141.625) (width 0.2) (layer "B.Cu") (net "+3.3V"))
 (segment (start 194.554 59.092732) (end 193.670267 58.209) (width 0.2) (layer "B.Cu") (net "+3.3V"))
 (segment (start 214.752387 143.395) (end 218.86 139.287387) (width 0.2) (layer "B.Cu") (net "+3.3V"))
 (segment (start 209.259315 143.395) (end 214.752387 143.395) (width 0.2) (layer "B.Cu") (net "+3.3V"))
 (segment (start 218.86 96.51) (end 194.554 72.204) (width 0.2) (layer "B.Cu") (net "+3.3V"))
 (segment (start 206.5 140.635685) (end 209.259315 143.395) (width 0.2) (layer "B.Cu") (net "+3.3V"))
 (segment (start 176.611 58.209) (end 175.2225 59.5975) (width 0.2) (layer "B.Cu") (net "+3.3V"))
 (segment (start 194.554 72.204) (end 194.554 59.092732) (width 0.2) (layer "B.Cu") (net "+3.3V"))
 (segment (start 175.2225 59.5975) (end 177.86 62.235) (width 0.2) (layer "B.Cu") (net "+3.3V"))
 (segment (start 210.6 141.82) (end 210.6 136.586547) (width 0.2) (layer "B.Cu") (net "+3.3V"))
 (segment (start 193.670267 58.209) (end 176.611 58.209) (width 0.2) (layer "B.Cu") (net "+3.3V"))
 (segment (start 151.79 99.07) (end 151.79 137.49) (width 0.2) (layer "B.Cu") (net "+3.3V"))
 (segment (start 176.3 63.795) (end 176.3 74.56) (width 0.2) (layer "B.Cu") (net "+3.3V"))
 (segment (start 206.5 135.786547) (end 206.5 140.635685) (width 0.2) (layer "B.Cu") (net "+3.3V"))
 (segment (start 187.72 109.296547) (end 187.72 90.9) (width 0.2) (layer "B.Cu") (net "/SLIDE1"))
 (segment (start 185.58 90.9) (end 183.6 88.92) (width 0.2) (layer "B.Cu") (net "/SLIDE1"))
 (segment (start 183.6 69.195) (end 193.1 59.695) (width 0.2) (layer "B.Cu") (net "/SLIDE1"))
 (segment (start 159.425 137.591547) (end 187.72 109.296547) (width 0.2) (layer "B.Cu") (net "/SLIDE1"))
 (segment (start 187.72 90.9) (end 185.58 90.9) (width 0.2) (layer "B.Cu") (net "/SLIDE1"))
 (segment (start 183.6 88.92) (end 183.6 69.195) (width 0.2) (layer "B.Cu") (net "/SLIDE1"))
 (segment (start 159.425 141.625) (end 159.425 137.591547) (width 0.2) (layer "B.Cu") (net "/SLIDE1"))
 (segment (start 193.1 72.395) (end 194.554 73.849) (width 0.2) (layer "F.Cu") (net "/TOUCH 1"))
 (segment (start 185 113.32376) (end 185 120) (width 0.2) (layer "F.Cu") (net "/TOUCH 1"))
 (segment (start 194.554 73.849) (end 194.554 95.446) (width 0.2) (layer "F.Cu") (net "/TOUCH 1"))
 (segment (start 194.554 95.446) (end 192.525 97.475) (width 0.2) (layer "F.Cu") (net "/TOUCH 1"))
 (segment (start 192.525 97.475) (end 192.525 105.79876) (width 0.2) (layer "F.Cu") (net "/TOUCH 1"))
 (segment (start 192.525 105.79876) (end 185 113.32376) (width 0.2) (layer "F.Cu") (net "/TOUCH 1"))
 (segment (start 177.7 116.97624) (end 177.7 129.7) (width 0.2) (layer "F.Cu") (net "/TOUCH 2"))
 (segment (start 177.7 107.234314) (end 179.1 108.634314) (width 0.2) (layer "F.Cu") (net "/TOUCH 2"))
 (segment (start 178.525 94.9) (end 178.525 95.9) (width 0.2) (layer "F.Cu") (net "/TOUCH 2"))
 (segment (start 175.975 92.35) (end 178.525 94.9) (width 0.2) (layer "F.Cu") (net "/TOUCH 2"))
 (segment (start 177.7 96.725) (end 177.7 107.234314) (width 0.2) (layer "F.Cu") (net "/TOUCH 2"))
 (segment (start 177.86 69.855) (end 175.975 71.74) (width 0.2) (layer "F.Cu") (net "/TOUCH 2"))
 (segment (start 179.1 115.57624) (end 177.7 116.97624) (width 0.2) (layer "F.Cu") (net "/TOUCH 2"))
 (segment (start 179.1 108.634314) (end 179.1 115.57624) (width 0.2) (layer "F.Cu") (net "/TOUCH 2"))
 (segment (start 185 130.32376) (end 185 137) (width 0.2) (layer "F.Cu") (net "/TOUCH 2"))
 (segment (start 178.525 95.9) (end 177.7 96.725) (width 0.2) (layer "F.Cu") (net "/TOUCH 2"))
 (segment (start 175.975 71.74) (end 175.975 92.35) (width 0.2) (layer "F.Cu") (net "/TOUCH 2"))
 (segment (start 177.7 129.7) (end 185 137) (width 0.2) (layer "F.Cu") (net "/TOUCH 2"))
 (segment (start 195.125 96.6) (end 193.05 98.675) (width 0.2) (layer "F.Cu") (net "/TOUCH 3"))
 (segment (start 192.42 107.505) (end 192.42 121.2) (width 0.2) (layer "F.Cu") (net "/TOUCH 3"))
 (segment (start 193.1 69.855) (end 195.125 71.88) (width 0.2) (layer "F.Cu") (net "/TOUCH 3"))
 (segment (start 193.05 106.875) (end 192.42 107.505) (width 0.2) (layer "F.Cu") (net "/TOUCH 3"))
 (segment (start 193.05 98.675) (end 193.05 106.875) (width 0.2) (layer "F.Cu") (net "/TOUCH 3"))
 (segment (start 192.42 121.2) (end 199.72 128.5) (width 0.2) (layer "F.Cu") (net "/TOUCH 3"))
 (segment (start 195.125 71.88) (end 195.125 96.6) (width 0.2) (layer "F.Cu") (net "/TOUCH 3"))
 (segment (start 195.625 69.84) (end 195.625 107.405) (width 0.2) (layer "F.Cu") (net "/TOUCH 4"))
 (segment (start 193.1 67.315) (end 195.625 69.84) (width 0.2) (layer "F.Cu") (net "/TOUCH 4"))
 (segment (start 195.625 107.405) (end 199.72 111.5) (width 0.2) (layer "F.Cu") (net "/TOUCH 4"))
 (segment (start 194.154 75.989) (end 194.154 93.846) (width 0.2) (layer "F.Cu") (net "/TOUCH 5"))
 (segment (start 194.154 93.846) (end 185 103) (width 0.2) (layer "F.Cu") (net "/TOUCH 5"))
 (segment (start 193.1 74.935) (end 194.154 75.989) (width 0.2) (layer "F.Cu") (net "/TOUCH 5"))
 (segment (start 170.28 102.67) (end 170.28 111.5) (width 0.2) (layer "F.Cu") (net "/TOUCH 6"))
 (segment (start 175.075 93.275) (end 177.375 95.575) (width 0.2) (layer "F.Cu") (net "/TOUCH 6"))
 (segment (start 175.075 67.56) (end 175.075 93.275) (width 0.2) (layer "F.Cu") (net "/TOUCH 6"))
 (segment (start 176.7425 66.1975) (end 177.86 67.315) (width 0.2) (layer "F.Cu") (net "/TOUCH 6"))
 (segment (start 176.7425 65.8925) (end 175.075 67.56) (width 0.2) (layer "F.Cu") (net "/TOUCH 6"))
 (segment (start 176.7425 65.8925) (end 176.7425 66.1975) (width 0.2) (layer "F.Cu") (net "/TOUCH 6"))
 (segment (start 177.375 95.575) (end 170.28 102.67) (width 0.2) (layer "F.Cu") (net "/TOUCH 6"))
 (segment (start 177.675 114.42876) (end 173.30376 118.8) (width 0.2) (layer "F.Cu") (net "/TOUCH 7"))
 (segment (start 175.475 92.925) (end 178.075 95.525) (width 0.2) (layer "F.Cu") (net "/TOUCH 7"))
 (segment (start 178.914 65.829) (end 177.86 64.775) (width 0.2) (layer "F.Cu") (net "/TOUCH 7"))
 (segment (start 172.175 128.5) (end 170.28 128.5) (width 0.2) (layer "F.Cu") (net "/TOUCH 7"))
 (segment (start 177.27 68.26) (end 177.379 68.369) (width 0.2) (layer "F.Cu") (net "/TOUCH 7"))
 (segment (start 173.30376 118.8) (end 173.175 118.8) (width 0.2) (layer "F.Cu") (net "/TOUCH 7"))
 (segment (start 176.635 68.54) (end 175.475 69.7) (width 0.2) (layer "F.Cu") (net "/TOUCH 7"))
 (segment (start 171.775 120.2) (end 171.775 128.1) (width 0.2) (layer "F.Cu") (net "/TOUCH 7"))
 (segment (start 175.925 97.675) (end 175.925 106.025) (width 0.2) (layer "F.Cu") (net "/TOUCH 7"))
 (segment (start 178.296582 68.369) (end 178.914 67.751582) (width 0.2) (layer "F.Cu") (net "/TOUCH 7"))
 (segment (start 175.475 69.7) (end 175.475 92.925) (width 0.2) (layer "F.Cu") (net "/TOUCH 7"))
 (segment (start 177.379 68.369) (end 178.296582 68.369) (width 0.2) (layer "F.Cu") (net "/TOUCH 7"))
 (segment (start 178.075 95.525) (end 175.925 97.675) (width 0.2) (layer "F.Cu") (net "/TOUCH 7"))
 (segment (start 177.27 68.26) (end 176.99 68.54) (width 0.2) (layer "F.Cu") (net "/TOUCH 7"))
 (segment (start 178.914 67.751582) (end 178.914 65.829) (width 0.2) (layer "F.Cu") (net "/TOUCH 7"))
 (segment (start 175.925 106.025) (end 177.675 107.775) (width 0.2) (layer "F.Cu") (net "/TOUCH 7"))
 (segment (start 177.675 107.775) (end 177.675 114.42876) (width 0.2) (layer "F.Cu") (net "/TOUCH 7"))
 (segment (start 176.99 68.54) (end 176.635 68.54) (width 0.2) (layer "F.Cu") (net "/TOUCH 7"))
 (segment (start 171.775 128.1) (end 172.175 128.5) (width 0.2) (layer "F.Cu") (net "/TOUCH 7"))
 (segment (start 173.175 118.8) (end 171.775 120.2) (width 0.2) (layer "F.Cu") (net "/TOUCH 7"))
 (segment (start 218.46 97.23) (end 194.154 72.924) (width 0.2) (layer "B.Cu") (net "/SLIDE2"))
 (segment (start 192.046 67.751582) (end 192.046 66.878418) (width 0.2) (layer "B.Cu") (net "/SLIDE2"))
 (segment (start 214.1 141.82) (end 214.9 141.02) (width 0.2) (layer "B.Cu") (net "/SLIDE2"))
 (segment (start 192.663418 68.369) (end 192.046 67.751582) (width 0.2) (layer "B.Cu") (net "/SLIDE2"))
 (segment (start 193.1 64.775) (end 193.1 64.95) (width 0.2) (layer "B.Cu") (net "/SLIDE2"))
 (segment (start 194.154 72.924) (end 194.154 69.418418) (width 0.2) (layer "B.Cu") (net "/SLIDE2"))
 (segment (start 194.154 69.418418) (end 193.104582 68.369) (width 0.2) (layer "B.Cu") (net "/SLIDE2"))
 (segment (start 214.9 141.02) (end 214.9 136.986547) (width 0.2) (layer "B.Cu") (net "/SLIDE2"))
 (segment (start 193.1 65.824418) (end 193.1 64.775) (width 0.2) (layer "B.Cu") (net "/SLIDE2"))
 (segment (start 193.104582 68.369) (end 192.663418 68.369) (width 0.2) (layer "B.Cu") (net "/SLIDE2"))
 (segment (start 218.46 133.426547) (end 218.46 97.23) (width 0.2) (layer "B.Cu") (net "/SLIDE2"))
 (segment (start 192.046 66.878418) (end 193.1 65.824418) (width 0.2) (layer "B.Cu") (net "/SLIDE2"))
 (segment (start 214.9 136.986547) (end 218.46 133.426547) (width 0.2) (layer "B.Cu") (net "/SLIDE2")))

